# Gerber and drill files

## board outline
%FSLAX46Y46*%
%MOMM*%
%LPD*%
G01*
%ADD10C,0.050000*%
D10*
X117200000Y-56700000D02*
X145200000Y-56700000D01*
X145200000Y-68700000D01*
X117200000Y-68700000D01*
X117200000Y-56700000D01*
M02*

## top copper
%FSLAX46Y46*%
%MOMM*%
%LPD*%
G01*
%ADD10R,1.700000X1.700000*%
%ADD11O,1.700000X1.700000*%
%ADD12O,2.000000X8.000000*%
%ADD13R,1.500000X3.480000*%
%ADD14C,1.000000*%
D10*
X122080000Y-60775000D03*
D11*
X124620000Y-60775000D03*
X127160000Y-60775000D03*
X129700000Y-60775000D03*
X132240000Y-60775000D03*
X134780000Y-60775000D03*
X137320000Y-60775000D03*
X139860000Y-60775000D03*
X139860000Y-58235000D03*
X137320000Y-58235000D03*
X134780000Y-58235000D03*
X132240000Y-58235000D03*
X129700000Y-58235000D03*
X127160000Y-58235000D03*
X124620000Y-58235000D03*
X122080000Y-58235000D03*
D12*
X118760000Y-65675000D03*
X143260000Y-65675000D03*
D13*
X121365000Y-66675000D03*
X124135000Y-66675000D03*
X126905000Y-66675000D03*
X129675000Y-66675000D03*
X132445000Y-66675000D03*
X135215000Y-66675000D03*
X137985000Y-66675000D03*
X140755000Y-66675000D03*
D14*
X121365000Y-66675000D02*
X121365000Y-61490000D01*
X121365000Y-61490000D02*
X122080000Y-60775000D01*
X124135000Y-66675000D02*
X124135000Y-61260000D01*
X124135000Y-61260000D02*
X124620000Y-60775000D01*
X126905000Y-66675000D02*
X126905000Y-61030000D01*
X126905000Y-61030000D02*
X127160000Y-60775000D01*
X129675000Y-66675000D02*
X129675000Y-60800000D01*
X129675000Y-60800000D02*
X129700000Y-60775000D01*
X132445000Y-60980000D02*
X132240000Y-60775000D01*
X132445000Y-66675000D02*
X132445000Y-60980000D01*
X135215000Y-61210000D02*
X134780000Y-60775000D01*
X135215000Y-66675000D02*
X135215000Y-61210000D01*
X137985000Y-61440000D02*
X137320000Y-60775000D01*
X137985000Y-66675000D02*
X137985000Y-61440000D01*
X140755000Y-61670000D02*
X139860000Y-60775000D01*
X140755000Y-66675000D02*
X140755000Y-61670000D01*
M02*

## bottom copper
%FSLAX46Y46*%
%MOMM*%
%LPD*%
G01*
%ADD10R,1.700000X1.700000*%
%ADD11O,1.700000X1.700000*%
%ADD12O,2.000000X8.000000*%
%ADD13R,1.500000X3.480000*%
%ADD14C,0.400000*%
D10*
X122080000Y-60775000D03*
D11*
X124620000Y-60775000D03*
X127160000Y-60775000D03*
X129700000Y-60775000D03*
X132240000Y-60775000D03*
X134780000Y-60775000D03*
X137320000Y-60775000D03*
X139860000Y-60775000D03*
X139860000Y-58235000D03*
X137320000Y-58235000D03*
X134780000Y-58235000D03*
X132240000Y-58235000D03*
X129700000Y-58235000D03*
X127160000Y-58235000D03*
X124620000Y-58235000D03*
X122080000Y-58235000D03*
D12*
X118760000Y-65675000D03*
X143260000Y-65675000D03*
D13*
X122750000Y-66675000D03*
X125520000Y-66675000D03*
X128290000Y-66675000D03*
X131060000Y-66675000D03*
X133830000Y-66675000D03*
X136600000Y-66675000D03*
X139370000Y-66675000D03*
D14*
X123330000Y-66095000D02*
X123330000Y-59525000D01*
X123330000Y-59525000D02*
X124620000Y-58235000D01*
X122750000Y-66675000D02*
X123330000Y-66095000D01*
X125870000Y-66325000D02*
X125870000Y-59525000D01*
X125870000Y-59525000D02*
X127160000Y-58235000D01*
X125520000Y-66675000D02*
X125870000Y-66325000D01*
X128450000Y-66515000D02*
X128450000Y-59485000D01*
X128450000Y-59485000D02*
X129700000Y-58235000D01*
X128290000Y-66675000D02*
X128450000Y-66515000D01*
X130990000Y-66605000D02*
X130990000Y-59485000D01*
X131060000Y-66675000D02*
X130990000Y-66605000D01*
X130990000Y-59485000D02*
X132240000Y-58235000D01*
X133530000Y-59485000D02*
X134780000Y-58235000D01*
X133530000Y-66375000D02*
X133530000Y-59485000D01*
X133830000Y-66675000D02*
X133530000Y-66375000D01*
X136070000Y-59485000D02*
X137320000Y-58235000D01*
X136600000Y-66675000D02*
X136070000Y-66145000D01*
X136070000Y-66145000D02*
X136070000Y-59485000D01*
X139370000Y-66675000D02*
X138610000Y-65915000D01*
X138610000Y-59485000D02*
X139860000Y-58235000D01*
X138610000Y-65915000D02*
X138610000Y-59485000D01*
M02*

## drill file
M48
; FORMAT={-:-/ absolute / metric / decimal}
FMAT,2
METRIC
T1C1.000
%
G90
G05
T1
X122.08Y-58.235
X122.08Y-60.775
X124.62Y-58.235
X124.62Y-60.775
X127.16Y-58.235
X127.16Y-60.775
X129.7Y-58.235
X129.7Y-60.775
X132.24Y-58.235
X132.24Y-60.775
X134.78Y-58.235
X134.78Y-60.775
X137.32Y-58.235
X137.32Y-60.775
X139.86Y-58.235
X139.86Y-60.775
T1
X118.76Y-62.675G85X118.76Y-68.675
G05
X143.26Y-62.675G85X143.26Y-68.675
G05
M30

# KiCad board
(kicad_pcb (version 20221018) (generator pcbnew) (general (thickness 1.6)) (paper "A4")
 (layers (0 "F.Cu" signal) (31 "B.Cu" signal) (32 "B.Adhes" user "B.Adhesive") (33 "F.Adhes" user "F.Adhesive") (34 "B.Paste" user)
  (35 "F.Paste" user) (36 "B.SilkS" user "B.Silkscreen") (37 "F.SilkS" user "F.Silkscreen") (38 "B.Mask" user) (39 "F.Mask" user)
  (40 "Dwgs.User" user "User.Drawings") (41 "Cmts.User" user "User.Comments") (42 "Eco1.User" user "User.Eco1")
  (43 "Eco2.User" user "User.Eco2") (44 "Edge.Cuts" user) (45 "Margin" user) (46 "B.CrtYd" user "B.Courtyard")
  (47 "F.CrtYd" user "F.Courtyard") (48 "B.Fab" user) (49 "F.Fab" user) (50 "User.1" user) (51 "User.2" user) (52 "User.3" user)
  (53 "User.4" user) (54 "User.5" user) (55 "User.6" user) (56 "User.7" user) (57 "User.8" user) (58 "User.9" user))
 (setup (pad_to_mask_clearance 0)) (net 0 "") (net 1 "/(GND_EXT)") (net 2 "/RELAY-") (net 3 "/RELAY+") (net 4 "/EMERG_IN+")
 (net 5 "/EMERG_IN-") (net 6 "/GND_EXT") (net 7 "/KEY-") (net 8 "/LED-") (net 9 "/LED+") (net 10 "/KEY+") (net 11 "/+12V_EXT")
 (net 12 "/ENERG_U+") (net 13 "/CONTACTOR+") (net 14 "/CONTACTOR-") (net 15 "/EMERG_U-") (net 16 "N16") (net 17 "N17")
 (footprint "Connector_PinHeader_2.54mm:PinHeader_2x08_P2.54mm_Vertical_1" (layer "F.Cu") (at 122.08 60.775 90)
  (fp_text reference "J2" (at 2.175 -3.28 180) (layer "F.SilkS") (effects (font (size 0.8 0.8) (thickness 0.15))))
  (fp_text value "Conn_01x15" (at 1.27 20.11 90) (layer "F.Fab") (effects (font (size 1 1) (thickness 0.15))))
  (pad "1" thru_hole rect (at 0 0 90) (size 1.7 1.7) (drill 1) (layers "*.Cu" "*.Mask") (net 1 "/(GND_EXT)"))
  (pad "2" thru_hole oval (at 0 2.54 90) (size 1.7 1.7) (drill 1) (layers "*.Cu" "*.Mask") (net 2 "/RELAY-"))
  (pad "3" thru_hole oval (at 0 5.08 90) (size 1.7 1.7) (drill 1) (layers "*.Cu" "*.Mask") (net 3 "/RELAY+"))
  (pad "4" thru_hole oval (at 0 7.62 90) (size 1.7 1.7) (drill 1) (layers "*.Cu" "*.Mask") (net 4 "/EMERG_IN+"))
  (pad "5" thru_hole oval (at 0 10.16 90) (size 1.7 1.7) (drill 1) (layers "*.Cu" "*.Mask") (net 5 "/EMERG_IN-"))
  (pad "6" thru_hole oval (at 0 12.7 90) (size 1.7 1.7) (drill 1) (layers "*.Cu" "*.Mask") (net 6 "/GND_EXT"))
  (pad "7" thru_hole oval (at 0 15.24 90) (size 1.7 1.7) (drill 1) (layers "*.Cu" "*.Mask") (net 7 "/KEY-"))
  (pad "8" thru_hole oval (at 0 17.78 90) (size 1.7 1.7) (drill 1) (layers "*.Cu" "*.Mask") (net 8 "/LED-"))
  (pad "9" thru_hole oval (at 2.54 17.78 90) (size 1.7 1.7) (drill 1) (layers "*.Cu" "*.Mask") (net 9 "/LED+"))
  (pad "10" thru_hole oval (at 2.54 15.24 90) (size 1.7 1.7) (drill 1) (layers "*.Cu" "*.Mask") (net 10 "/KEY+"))
  (pad "11" thru_hole oval (at 2.54 12.7 90) (size 1.7 1.7) (drill 1) (layers "*.Cu" "*.Mask") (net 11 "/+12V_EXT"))
  (pad "12" thru_hole oval (at 2.54 10.16 90) (size 1.7 1.7) (drill 1) (layers "*.Cu" "*.Mask") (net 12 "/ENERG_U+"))
  (pad "13" thru_hole oval (at 2.54 7.62 90) (size 1.7 1.7) (drill 1) (layers "*.Cu" "*.Mask") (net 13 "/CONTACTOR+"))
  (pad "14" thru_hole oval (at 2.54 5.08 90) (size 1.7 1.7) (drill 1) (layers "*.Cu" "*.Mask") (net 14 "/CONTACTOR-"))
  (pad "15" thru_hole oval (at 2.54 2.54 90) (size 1.7 1.7) (drill 1) (layers "*.Cu" "*.Mask") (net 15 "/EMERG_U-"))
  (pad "16" thru_hole oval (at 2.54 0 90) (size 1.7 1.7) (drill 1) (layers "*.Cu" "*.Mask") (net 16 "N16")))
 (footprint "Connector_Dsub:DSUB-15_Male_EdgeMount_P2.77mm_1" (layer "F.Cu") (at 131.06 66.675)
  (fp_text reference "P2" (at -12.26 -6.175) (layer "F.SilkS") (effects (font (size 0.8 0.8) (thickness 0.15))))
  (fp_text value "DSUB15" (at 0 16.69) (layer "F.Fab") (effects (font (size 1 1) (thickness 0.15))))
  (pad "0" thru_hole oval (at -12.3 -1) (size 2 8) (drill oval 1 7) (layers "*.Cu" "*.Mask") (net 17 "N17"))
  (pad "0" thru_hole oval (at 12.2 -1) (size 2 8) (drill oval 1 7) (layers "*.Cu" "*.Mask") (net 17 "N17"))
  (pad "1" smd rect (at -9.695 0) (size 1.5 3.48) (layers "F.Cu" "F.Paste" "F.Mask") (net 1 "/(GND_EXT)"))
  (pad "2" smd rect (at -6.925 0) (size 1.5 3.48) (layers "F.Cu" "F.Paste" "F.Mask") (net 2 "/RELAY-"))
  (pad "3" smd rect (at -4.155 0) (size 1.5 3.48) (layers "F.Cu" "F.Paste" "F.Mask") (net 3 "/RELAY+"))
  (pad "4" smd rect (at -1.385 0) (size 1.5 3.48) (layers "F.Cu" "F.Paste" "F.Mask") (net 4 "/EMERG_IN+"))
  (pad "5" smd rect (at 1.385 0) (size 1.5 3.48) (layers "F.Cu" "F.Paste" "F.Mask") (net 5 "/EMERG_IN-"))
  (pad "6" smd rect (at 4.155 0) (size 1.5 3.48) (layers "F.Cu" "F.Paste" "F.Mask") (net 6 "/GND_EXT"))
  (pad "7" smd rect (at 6.925 0) (size 1.5 3.48) (layers "F.Cu" "F.Paste" "F.Mask") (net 7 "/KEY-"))
  (pad "8" smd rect (at 9.695 0) (size 1.5 3.48) (layers "F.Cu" "F.Paste" "F.Mask") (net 8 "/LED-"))
  (pad "9" smd rect (at -8.31 0) (size 1.5 3.48) (layers "B.Cu" "B.Paste" "B.Mask") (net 15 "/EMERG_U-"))
  (pad "10" smd rect (at -5.54 0) (size 1.5 3.48) (layers "B.Cu" "B.Paste" "B.Mask") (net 14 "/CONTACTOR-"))
  (pad "11" smd rect (at -2.77 0) (size 1.5 3.48) (layers "B.Cu" "B.Paste" "B.Mask") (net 13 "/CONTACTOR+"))
  (pad "12" smd rect (at 0 0) (size 1.5 3.48) (layers "B.Cu" "B.Paste" "B.Mask") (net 12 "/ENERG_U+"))
  (pad "13" smd rect (at 2.77 0) (size 1.5 3.48) (layers "B.Cu" "B.Paste" "B.Mask") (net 11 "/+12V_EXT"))
  (pad "14" smd rect (at 5.54 0) (size 1.5 3.48) (layers "B.Cu" "B.Paste" "B.Mask") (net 10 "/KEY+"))
  (pad "15" smd rect (at 8.31 0) (size 1.5 3.48) (layers "B.Cu" "B.Paste" "B.Mask") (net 9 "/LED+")))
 (gr_rect (start 117.2 56.7) (end 145.2 68.7) (stroke (width 0.05) (type default)) (fill none) (layer "Edge.Cuts"))
 (segment (start 121.365 66.675) (end 121.365 61.49) (width 1) (layer "F.Cu") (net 1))
 (segment (start 121.365 61.49) (end 122.08 60.775) (width 1) (layer "F.Cu") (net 1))
 (segment (start 124.135 66.675) (end 124.135 61.26) (width 1) (layer "F.Cu") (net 2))
 (segment (start 124.135 61.26) (end 124.62 60.775) (width 1) (layer "F.Cu") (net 2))
 (segment (start 126.905 66.675) (end 126.905 61.03) (width 1) (layer "F.Cu") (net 3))
 (segment (start 126.905 61.03) (end 127.16 60.775) (width 1) (layer "F.Cu") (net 3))
 (segment (start 129.675 66.675) (end 129.675 60.8) (width 1) (layer "F.Cu") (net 4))
 (segment (start 129.675 60.8) (end 129.7 60.775) (width 1) (layer "F.Cu") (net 4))
 (segment (start 132.445 60.98) (end 132.24 60.775) (width 1) (layer "F.Cu") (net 5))
 (segment (start 132.445 66.675) (end 132.445 60.98) (width 1) (layer "F.Cu") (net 5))
 (segment (start 135.215 61.21) (end 134.78 60.775) (width 1) (layer "F.Cu") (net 6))
 (segment (start 135.215 66.675) (end 135.215 61.21) (width 1) (layer "F.Cu") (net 6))
 (segment (start 137.985 61.44) (end 137.32 60.775) (width 1) (layer "F.Cu") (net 7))
 (segment (start 137.985 66.675) (end 137.985 61.44) (width 1) (layer "F.Cu") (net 7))
 (segment (start 140.755 61.67) (end 139.86 60.775) (width 1) (layer "F.Cu") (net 8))
 (segment (start 140.755 66.675) (end 140.755 61.67) (width 1) (layer "F.Cu") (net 8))
 (segment (start 123.33 66.095) (end 123.33 59.525) (width 0.4) (layer "B.Cu") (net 15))
 (segment (start 123.33 59.525) (end 124.62 58.235) (width 0.4) (layer "B.Cu") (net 15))
 (segment (start 122.75 66.675) (end 123.33 66.095) (width 0.4) (layer "B.Cu") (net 15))
 (segment (start 125.87 66.325) (end 125.87 59.525) (width 0.4) (layer "B.Cu") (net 14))
 (segment (start 125.87 59.525) (end 127.16 58.235) (width 0.4) (layer "B.Cu") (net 14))
 (segment (start 125.52 66.675) (end 125.87 66.325) (width 0.4) (layer "B.Cu") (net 14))
 (segment (start 128.45 66.515) (end 128.45 59.485) (width 0.4) (layer "B.Cu") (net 13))
 (segment (start 128.45 59.485) (end 129.7 58.235) (width 0.4) (layer "B.Cu") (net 13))
 (segment (start 128.29 66.675) (end 128.45 66.515) (width 0.4) (layer "B.Cu") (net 13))
 (segment (start 130.99 66.605) (end 130.99 59.485) (width 0.4) (layer "B.Cu") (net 12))
 (segment (start 131.06 66.675) (end 130.99 66.605) (width 0.4) (layer "B.Cu") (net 12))
 (segment (start 130.99 59.485) (end 132.24 58.235) (width 0.4) (layer "B.Cu") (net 12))
 (segment (start 133.53 59.485) (end 134.78 58.235) (width 0.4) (layer "B.Cu") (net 11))
 (segment (start 133.53 66.375) (end 133.53 59.485) (width 0.4) (layer "B.Cu") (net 11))
 (segment (start 133.83 66.675) (end 133.53 66.375) (width 0.4) (layer "B.Cu") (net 11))
 (segment (start 136.07 59.485) (end 137.32 58.235) (width 0.4) (layer "B.Cu") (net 10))
 (segment (start 136.6 66.675) (end 136.07 66.145) (width 0.4) (layer "B.Cu") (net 10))
 (segment (start 136.07 66.145) (end 136.07 59.485) (width 0.4) (layer "B.Cu") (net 10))
 (segment (start 139.37 66.675) (end 138.61 65.915) (width 0.4) (layer "B.Cu") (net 9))
 (segment (start 138.61 59.485) (end 139.86 58.235) (width 0.4) (layer "B.Cu") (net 9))
 (segment (start 138.61 65.915) (end 138.61 59.485) (width 0.4) (layer "B.Cu") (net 9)))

